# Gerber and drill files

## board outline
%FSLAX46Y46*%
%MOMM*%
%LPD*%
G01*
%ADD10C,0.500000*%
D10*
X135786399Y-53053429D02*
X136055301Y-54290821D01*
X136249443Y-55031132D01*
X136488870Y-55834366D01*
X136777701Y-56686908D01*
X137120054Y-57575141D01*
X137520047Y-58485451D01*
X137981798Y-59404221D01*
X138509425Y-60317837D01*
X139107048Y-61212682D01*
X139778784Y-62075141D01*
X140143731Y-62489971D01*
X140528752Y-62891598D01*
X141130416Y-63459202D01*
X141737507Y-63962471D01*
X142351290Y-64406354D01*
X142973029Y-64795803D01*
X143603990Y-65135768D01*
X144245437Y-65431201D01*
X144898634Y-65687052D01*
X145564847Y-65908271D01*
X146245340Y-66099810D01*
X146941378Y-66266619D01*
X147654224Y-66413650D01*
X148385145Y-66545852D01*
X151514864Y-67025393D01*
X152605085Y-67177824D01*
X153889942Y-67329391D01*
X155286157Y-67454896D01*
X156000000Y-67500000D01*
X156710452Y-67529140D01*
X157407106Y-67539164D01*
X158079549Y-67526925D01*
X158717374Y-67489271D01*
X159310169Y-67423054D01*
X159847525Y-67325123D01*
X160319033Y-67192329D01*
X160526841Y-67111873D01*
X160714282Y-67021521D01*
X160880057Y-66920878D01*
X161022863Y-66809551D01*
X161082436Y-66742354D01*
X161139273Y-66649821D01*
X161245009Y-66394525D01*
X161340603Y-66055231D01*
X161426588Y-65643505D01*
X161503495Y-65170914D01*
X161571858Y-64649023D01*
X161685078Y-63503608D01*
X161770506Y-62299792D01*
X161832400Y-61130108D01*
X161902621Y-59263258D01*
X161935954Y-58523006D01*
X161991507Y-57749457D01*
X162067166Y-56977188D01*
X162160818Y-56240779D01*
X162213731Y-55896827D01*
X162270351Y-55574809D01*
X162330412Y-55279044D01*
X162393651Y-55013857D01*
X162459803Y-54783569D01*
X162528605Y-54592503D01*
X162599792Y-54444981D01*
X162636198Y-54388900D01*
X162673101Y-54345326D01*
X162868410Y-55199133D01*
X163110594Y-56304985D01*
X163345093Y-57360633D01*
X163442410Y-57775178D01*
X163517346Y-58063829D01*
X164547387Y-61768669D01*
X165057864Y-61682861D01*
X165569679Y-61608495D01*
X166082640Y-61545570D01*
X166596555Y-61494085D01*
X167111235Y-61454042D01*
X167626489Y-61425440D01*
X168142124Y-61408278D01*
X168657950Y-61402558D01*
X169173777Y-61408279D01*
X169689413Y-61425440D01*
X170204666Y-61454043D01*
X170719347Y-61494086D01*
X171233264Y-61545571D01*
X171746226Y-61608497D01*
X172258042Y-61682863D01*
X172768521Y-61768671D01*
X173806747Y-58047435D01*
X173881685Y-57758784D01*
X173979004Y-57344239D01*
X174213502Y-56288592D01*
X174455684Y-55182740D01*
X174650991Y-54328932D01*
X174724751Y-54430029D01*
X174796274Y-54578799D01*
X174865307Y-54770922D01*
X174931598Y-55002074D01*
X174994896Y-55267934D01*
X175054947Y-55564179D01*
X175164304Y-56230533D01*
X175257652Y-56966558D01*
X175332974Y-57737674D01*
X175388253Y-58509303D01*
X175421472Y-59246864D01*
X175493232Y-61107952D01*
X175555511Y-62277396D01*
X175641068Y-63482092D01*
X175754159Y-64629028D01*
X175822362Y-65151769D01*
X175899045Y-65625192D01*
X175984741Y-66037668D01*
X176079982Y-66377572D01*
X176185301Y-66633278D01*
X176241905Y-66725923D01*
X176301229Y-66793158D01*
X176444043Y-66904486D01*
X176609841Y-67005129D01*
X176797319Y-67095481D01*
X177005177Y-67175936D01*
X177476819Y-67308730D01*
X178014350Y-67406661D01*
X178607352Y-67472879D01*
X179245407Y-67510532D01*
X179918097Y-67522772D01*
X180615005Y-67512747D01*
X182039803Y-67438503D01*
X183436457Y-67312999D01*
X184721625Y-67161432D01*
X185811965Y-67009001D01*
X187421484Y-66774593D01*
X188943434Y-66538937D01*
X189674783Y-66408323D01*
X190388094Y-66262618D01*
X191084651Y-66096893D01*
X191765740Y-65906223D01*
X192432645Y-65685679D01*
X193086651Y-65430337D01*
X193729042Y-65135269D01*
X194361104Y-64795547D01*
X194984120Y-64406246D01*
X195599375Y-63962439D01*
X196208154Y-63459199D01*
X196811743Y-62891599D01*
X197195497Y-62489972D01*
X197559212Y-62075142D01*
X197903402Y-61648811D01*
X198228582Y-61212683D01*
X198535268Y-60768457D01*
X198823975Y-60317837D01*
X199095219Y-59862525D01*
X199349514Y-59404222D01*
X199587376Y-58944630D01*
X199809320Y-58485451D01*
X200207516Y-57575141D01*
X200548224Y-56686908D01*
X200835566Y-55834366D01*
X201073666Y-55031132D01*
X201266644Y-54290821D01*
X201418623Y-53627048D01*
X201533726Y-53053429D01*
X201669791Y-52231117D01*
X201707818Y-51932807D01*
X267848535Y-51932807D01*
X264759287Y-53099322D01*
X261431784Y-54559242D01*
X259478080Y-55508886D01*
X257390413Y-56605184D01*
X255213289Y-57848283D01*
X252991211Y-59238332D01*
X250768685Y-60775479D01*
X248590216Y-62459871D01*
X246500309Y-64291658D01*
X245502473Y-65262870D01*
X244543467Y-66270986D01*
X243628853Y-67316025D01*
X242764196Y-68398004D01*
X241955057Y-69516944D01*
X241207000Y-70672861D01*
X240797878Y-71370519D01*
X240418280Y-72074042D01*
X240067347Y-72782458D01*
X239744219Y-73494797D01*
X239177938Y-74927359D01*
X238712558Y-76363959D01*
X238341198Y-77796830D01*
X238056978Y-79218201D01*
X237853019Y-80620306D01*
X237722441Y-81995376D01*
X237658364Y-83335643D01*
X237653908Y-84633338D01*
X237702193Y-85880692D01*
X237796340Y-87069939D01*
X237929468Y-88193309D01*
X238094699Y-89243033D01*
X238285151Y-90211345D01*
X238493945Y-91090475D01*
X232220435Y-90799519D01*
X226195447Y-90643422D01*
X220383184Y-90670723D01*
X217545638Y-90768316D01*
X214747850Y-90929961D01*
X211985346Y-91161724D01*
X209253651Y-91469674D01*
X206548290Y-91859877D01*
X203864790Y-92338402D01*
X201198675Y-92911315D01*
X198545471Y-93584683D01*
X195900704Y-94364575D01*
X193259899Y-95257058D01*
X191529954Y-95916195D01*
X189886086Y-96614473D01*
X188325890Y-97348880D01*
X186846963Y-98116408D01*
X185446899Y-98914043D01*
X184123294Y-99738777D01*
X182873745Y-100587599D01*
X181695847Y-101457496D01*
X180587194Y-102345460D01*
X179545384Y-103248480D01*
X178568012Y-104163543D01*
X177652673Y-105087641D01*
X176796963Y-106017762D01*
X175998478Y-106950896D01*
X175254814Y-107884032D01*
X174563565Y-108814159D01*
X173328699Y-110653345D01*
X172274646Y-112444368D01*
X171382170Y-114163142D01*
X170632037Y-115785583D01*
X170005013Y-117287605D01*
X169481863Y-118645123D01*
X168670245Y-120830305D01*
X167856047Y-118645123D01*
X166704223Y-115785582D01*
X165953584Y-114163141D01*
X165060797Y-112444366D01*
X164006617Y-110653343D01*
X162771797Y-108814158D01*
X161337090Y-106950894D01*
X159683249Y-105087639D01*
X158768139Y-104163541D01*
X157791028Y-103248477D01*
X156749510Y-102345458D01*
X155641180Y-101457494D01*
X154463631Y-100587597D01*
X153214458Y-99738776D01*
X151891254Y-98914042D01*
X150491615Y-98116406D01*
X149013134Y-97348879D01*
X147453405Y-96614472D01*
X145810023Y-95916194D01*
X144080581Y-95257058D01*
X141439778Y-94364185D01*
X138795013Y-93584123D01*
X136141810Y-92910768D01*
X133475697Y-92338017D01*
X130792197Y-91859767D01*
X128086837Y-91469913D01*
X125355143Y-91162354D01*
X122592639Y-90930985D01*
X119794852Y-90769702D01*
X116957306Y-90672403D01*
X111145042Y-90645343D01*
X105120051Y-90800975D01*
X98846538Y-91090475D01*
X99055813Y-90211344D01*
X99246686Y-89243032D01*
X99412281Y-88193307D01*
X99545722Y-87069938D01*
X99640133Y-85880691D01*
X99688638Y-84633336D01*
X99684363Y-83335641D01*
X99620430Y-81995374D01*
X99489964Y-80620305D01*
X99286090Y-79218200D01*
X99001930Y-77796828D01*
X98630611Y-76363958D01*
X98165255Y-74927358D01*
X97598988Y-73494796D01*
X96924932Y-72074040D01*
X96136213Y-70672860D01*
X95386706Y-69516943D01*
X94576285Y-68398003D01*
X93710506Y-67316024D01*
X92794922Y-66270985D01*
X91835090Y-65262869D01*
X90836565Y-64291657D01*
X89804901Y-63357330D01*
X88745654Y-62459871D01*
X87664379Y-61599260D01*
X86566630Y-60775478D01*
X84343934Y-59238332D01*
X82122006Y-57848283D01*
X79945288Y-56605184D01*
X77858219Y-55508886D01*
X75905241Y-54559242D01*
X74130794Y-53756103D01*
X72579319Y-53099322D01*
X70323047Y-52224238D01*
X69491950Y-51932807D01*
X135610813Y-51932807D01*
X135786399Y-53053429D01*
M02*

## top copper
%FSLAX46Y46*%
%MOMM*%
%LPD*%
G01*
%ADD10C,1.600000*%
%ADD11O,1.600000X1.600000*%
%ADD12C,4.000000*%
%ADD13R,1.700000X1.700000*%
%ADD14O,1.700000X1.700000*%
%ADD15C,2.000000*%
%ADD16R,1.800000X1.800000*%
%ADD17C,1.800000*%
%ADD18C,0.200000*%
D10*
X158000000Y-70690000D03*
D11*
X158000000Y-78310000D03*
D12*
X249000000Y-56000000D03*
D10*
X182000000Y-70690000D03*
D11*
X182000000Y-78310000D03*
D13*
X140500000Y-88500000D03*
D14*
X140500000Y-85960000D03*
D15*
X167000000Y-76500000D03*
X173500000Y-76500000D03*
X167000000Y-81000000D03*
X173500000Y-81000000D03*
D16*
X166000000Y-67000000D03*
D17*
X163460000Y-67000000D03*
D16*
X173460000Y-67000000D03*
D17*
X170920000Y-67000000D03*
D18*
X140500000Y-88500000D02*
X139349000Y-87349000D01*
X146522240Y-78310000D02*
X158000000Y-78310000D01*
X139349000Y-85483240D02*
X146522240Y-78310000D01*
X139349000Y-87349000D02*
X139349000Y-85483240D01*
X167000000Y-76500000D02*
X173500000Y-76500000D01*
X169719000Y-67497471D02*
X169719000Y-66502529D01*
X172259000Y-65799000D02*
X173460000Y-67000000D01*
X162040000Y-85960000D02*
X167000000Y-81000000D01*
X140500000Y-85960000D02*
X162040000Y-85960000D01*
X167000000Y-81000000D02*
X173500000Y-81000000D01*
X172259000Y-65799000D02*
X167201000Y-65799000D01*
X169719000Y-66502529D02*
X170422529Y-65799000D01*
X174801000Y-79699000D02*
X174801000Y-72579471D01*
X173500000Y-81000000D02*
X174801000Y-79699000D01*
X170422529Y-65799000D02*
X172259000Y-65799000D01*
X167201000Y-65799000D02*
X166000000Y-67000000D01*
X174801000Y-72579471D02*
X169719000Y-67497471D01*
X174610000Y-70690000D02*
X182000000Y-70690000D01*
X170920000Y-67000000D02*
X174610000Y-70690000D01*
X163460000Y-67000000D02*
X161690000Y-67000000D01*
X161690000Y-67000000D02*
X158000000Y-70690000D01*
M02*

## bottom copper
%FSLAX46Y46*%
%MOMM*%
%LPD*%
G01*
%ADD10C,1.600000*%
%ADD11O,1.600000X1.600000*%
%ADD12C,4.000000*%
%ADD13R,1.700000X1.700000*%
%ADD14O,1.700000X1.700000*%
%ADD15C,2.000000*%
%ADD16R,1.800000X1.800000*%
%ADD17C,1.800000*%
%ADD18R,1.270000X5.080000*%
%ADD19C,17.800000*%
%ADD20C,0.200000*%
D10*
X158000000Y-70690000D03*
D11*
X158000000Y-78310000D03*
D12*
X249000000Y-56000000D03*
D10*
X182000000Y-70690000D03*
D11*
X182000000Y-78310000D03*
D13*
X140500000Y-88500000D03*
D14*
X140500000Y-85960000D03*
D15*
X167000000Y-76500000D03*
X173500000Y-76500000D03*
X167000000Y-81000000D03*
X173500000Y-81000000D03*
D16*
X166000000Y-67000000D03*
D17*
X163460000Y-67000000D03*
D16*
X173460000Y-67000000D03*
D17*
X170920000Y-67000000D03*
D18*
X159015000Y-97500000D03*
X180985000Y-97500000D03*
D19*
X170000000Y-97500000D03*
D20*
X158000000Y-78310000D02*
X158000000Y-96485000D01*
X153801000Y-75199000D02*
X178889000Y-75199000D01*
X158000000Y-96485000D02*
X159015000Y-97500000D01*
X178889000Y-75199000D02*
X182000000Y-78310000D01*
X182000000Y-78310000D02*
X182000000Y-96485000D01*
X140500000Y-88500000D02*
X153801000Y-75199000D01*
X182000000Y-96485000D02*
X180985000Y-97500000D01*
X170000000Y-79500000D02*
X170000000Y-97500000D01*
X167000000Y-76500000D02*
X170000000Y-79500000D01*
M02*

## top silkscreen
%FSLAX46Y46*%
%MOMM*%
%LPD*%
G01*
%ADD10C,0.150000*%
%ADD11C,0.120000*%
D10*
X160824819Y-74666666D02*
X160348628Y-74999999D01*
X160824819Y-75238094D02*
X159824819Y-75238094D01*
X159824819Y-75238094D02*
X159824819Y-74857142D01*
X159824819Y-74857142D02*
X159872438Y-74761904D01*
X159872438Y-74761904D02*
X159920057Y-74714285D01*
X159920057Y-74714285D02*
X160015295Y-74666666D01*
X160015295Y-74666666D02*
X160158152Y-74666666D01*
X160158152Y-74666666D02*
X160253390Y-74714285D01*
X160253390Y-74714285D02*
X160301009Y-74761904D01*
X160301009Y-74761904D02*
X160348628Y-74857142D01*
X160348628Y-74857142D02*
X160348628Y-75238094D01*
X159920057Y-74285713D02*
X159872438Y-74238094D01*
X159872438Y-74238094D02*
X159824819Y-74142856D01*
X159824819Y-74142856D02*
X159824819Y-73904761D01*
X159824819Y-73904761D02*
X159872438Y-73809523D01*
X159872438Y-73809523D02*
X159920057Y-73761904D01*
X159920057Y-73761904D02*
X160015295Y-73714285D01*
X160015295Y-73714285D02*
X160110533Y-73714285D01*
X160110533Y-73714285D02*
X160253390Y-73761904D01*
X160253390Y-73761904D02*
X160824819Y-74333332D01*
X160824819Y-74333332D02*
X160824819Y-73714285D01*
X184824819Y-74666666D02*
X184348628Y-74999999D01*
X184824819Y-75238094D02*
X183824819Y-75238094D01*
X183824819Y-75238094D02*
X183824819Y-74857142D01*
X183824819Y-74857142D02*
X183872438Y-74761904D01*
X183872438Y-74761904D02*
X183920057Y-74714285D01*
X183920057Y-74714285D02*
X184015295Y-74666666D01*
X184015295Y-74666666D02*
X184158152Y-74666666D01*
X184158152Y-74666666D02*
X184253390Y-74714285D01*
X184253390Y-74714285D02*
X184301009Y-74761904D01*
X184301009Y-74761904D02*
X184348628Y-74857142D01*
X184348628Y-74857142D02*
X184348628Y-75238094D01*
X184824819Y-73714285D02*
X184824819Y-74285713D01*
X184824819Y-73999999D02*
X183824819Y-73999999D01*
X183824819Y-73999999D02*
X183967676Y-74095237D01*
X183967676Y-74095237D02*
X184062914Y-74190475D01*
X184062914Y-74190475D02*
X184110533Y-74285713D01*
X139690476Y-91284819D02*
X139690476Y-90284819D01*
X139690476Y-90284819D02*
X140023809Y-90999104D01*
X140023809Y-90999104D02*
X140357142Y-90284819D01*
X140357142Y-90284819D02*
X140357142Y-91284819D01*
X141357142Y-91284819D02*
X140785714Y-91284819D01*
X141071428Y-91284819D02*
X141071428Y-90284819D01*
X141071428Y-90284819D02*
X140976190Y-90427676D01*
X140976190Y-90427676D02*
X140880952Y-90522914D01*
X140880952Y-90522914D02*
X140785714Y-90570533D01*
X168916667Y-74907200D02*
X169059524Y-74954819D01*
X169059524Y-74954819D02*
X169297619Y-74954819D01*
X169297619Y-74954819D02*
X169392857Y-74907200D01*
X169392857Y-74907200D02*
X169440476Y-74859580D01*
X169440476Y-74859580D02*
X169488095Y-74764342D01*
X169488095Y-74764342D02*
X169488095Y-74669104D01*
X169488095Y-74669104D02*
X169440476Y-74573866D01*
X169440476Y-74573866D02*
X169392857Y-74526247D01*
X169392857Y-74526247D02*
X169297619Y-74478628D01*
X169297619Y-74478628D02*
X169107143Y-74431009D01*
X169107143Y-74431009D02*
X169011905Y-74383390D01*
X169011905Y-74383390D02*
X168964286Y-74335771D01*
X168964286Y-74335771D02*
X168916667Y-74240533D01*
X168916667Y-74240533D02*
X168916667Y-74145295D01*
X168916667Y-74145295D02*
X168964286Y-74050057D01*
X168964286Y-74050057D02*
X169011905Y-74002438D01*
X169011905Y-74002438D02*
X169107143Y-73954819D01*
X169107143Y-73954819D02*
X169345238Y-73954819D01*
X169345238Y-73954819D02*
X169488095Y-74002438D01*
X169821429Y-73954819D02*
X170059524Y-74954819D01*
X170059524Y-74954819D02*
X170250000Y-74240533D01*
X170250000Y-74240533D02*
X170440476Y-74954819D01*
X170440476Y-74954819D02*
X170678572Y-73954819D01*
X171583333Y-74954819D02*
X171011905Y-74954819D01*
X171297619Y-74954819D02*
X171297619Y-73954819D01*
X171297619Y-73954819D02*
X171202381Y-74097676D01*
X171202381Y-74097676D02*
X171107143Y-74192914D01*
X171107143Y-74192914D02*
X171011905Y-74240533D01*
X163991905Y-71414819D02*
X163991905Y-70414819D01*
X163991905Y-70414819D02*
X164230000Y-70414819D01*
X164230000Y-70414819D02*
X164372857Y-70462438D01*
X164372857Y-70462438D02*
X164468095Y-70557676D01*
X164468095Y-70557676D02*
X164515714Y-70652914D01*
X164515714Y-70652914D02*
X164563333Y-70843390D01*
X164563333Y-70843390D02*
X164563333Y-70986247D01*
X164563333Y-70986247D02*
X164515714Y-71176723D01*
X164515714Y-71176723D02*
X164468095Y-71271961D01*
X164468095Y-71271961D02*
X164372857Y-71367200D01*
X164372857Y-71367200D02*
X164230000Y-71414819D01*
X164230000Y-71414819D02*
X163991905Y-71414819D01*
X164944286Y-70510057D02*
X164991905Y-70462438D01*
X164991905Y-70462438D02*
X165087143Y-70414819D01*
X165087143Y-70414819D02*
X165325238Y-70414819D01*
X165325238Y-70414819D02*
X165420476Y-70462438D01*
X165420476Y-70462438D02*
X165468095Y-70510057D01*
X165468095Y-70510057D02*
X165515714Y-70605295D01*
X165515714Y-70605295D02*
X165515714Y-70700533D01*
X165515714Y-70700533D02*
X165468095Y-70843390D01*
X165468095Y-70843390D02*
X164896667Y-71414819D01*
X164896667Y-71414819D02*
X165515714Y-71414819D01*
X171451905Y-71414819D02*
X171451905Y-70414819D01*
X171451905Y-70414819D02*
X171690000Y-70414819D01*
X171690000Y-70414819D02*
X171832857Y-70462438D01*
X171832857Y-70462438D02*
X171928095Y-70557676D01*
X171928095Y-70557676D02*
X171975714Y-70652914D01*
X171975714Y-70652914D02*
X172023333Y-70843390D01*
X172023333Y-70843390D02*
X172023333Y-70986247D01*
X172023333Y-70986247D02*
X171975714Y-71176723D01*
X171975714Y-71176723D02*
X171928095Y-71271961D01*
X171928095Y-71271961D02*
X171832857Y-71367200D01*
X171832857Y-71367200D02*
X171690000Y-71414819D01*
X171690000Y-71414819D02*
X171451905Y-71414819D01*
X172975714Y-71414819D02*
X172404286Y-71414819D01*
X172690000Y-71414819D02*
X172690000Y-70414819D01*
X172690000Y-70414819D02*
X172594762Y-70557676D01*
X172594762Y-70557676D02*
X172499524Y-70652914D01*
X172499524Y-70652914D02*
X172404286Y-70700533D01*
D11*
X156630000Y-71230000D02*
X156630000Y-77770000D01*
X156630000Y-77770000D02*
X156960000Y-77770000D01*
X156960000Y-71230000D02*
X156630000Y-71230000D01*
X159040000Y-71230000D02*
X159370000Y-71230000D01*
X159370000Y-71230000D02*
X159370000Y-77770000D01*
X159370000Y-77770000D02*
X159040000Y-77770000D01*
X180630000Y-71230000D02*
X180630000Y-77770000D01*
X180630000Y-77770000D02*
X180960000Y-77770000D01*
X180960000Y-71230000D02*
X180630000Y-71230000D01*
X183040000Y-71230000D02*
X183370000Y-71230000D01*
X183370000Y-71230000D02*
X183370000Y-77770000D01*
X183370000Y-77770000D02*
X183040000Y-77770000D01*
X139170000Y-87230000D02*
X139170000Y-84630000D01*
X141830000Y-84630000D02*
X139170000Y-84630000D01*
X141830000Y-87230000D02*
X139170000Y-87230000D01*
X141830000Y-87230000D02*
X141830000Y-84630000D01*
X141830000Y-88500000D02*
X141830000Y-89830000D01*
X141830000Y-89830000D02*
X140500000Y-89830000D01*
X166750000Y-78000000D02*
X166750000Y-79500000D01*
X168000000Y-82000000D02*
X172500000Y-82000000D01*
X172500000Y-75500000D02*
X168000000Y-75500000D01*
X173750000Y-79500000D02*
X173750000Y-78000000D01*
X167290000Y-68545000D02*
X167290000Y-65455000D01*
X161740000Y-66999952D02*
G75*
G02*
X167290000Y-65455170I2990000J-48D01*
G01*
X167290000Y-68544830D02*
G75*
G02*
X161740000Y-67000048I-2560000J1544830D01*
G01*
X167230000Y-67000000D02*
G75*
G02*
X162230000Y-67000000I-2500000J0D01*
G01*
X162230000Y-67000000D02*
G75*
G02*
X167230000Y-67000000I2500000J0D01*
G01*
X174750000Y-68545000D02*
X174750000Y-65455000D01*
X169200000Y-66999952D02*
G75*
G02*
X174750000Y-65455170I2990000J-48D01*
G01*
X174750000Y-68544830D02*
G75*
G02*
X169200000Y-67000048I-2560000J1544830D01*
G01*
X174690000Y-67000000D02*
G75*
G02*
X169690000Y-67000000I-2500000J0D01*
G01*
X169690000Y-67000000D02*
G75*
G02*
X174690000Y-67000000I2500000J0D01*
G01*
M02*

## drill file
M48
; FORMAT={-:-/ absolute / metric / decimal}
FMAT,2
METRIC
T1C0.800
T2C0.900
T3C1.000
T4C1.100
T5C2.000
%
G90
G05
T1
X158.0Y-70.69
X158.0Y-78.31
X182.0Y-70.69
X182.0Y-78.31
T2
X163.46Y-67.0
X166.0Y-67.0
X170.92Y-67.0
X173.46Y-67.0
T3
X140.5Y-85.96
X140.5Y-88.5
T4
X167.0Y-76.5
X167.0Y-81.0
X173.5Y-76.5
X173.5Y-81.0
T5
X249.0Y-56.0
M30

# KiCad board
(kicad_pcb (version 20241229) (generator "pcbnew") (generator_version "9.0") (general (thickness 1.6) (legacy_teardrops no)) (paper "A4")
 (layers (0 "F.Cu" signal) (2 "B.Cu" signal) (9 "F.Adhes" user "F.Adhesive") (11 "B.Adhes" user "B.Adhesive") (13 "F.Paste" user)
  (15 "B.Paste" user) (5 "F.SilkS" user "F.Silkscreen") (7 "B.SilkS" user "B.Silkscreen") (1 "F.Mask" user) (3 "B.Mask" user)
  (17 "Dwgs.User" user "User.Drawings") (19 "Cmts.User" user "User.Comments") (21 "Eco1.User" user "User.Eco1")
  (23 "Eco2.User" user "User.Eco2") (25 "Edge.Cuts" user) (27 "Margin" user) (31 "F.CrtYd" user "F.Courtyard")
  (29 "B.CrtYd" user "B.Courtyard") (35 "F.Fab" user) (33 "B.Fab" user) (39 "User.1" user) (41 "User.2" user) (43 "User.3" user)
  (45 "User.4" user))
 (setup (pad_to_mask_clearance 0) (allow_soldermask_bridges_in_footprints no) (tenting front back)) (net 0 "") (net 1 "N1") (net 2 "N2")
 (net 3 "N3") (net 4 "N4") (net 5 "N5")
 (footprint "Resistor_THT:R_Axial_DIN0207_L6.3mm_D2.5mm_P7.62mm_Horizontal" (layer "F.Cu") (at 158 70.69 -90)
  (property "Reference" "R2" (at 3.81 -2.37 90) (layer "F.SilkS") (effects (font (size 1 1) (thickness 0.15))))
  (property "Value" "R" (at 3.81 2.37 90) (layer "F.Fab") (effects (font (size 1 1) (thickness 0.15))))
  (fp_line (start 0.54 1.37) (end 7.08 1.37) (stroke (width 0.12) (type solid)) (layer "F.SilkS"))
  (fp_line (start 7.08 1.37) (end 7.08 1.04) (stroke (width 0.12) (type solid)) (layer "F.SilkS"))
  (fp_line (start 0.54 1.04) (end 0.54 1.37) (stroke (width 0.12) (type solid)) (layer "F.SilkS"))
  (fp_line (start 0.54 -1.04) (end 0.54 -1.37) (stroke (width 0.12) (type solid)) (layer "F.SilkS"))
  (fp_line (start 0.54 -1.37) (end 7.08 -1.37) (stroke (width 0.12) (type solid)) (layer "F.SilkS"))
  (fp_line (start 7.08 -1.37) (end 7.08 -1.04) (stroke (width 0.12) (type solid)) (layer "F.SilkS"))
  (pad "1" thru_hole circle (at 0 0 270) (size 1.6 1.6) (drill 0.8) (layers "*.Cu" "*.Mask") (remove_unused_layers no) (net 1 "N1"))
  (pad "2" thru_hole oval (at 7.62 0 270) (size 1.6 1.6) (drill 0.8) (layers "*.Cu" "*.Mask") (remove_unused_layers no) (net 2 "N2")))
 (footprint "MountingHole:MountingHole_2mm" (layer "F.Cu") (at 249 56)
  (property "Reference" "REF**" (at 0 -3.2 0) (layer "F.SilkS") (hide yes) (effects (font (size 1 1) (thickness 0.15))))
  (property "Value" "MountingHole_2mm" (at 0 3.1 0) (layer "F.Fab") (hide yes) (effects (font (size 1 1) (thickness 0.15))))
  (pad "" np_thru_hole circle (at 0 0) (size 4 4) (drill 2) (layers "*.Cu" "*.Mask")))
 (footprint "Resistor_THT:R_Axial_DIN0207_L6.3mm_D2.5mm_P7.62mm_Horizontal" (layer "F.Cu") (at 182 70.69 -90)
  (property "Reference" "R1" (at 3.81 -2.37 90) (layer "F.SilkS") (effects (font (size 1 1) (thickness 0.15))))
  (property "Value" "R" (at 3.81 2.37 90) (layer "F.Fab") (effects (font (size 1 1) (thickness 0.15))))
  (fp_line (start 0.54 1.37) (end 7.08 1.37) (stroke (width 0.12) (type solid)) (layer "F.SilkS"))
  (fp_line (start 7.08 1.37) (end 7.08 1.04) (stroke (width 0.12) (type solid)) (layer "F.SilkS"))
  (fp_line (start 0.54 1.04) (end 0.54 1.37) (stroke (width 0.12) (type solid)) (layer "F.SilkS"))
  (fp_line (start 0.54 -1.04) (end 0.54 -1.37) (stroke (width 0.12) (type solid)) (layer "F.SilkS"))
  (fp_line (start 0.54 -1.37) (end 7.08 -1.37) (stroke (width 0.12) (type solid)) (layer "F.SilkS"))
  (fp_line (start 7.08 -1.37) (end 7.08 -1.04) (stroke (width 0.12) (type solid)) (layer "F.SilkS"))
  (pad "1" thru_hole circle (at 0 0 270) (size 1.6 1.6) (drill 0.8) (layers "*.Cu" "*.Mask") (remove_unused_layers no) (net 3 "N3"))
  (pad "2" thru_hole oval (at 7.62 0 270) (size 1.6 1.6) (drill 0.8) (layers "*.Cu" "*.Mask") (remove_unused_layers no) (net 2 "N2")))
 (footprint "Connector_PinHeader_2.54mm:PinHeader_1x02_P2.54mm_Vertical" (layer "F.Cu") (at 140.5 88.5 180)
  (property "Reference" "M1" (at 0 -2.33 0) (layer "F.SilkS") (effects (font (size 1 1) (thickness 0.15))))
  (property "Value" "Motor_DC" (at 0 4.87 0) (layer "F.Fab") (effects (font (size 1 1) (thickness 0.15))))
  (fp_line (start 1.33 1.27) (end 1.33 3.87) (stroke (width 0.12) (type solid)) (layer "F.SilkS"))
  (fp_line (start -1.33 3.87) (end 1.33 3.87) (stroke (width 0.12) (type solid)) (layer "F.SilkS"))
  (fp_line (start -1.33 1.27) (end 1.33 1.27) (stroke (width 0.12) (type solid)) (layer "F.SilkS"))
  (fp_line (start -1.33 1.27) (end -1.33 3.87) (stroke (width 0.12) (type solid)) (layer "F.SilkS"))
  (fp_line (start -1.33 0) (end -1.33 -1.33) (stroke (width 0.12) (type solid)) (layer "F.SilkS"))
  (fp_line (start -1.33 -1.33) (end 0 -1.33) (stroke (width 0.12) (type solid)) (layer "F.SilkS"))
  (pad "1" thru_hole rect (at 0 0 180) (size 1.7 1.7) (drill 1) (layers "*.Cu" "*.Mask") (remove_unused_layers no) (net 2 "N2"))
  (pad "2" thru_hole oval (at 0 2.54 180) (size 1.7 1.7) (drill 1) (layers "*.Cu" "*.Mask") (remove_unused_layers no) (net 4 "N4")))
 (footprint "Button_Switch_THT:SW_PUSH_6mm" (layer "F.Cu") (at 167 76.5)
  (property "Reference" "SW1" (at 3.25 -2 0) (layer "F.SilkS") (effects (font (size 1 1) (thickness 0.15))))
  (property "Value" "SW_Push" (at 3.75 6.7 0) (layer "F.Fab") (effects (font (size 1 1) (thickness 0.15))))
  (fp_line (start -0.25 1.5) (end -0.25 3) (stroke (width 0.12) (type solid)) (layer "F.SilkS"))
  (fp_line (start 1 5.5) (end 5.5 5.5) (stroke (width 0.12) (type solid)) (layer "F.SilkS"))
  (fp_line (start 5.5 -1) (end 1 -1) (stroke (width 0.12) (type solid)) (layer "F.SilkS"))
  (fp_line (start 6.75 3) (end 6.75 1.5) (stroke (width 0.12) (type solid)) (layer "F.SilkS"))
  (pad "1" thru_hole circle (at 0 0 90) (size 2 2) (drill 1.1) (layers "*.Cu" "*.Mask") (remove_unused_layers no) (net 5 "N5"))
  (pad "1" thru_hole circle (at 6.5 0 90) (size 2 2) (drill 1.1) (layers "*.Cu" "*.Mask") (remove_unused_layers no) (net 5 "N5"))
  (pad "2" thru_hole circle (at 0 4.5 90) (size 2 2) (drill 1.1) (layers "*.Cu" "*.Mask") (remove_unused_layers no) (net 4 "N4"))
  (pad "2" thru_hole circle (at 6.5 4.5 90) (size 2 2) (drill 1.1) (layers "*.Cu" "*.Mask") (remove_unused_layers no) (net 4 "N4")))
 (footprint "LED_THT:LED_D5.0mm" (layer "F.Cu") (at 166 67 180)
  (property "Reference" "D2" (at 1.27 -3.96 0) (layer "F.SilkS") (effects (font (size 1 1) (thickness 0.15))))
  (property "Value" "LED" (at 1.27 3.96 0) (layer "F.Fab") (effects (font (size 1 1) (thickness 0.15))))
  (fp_line (start -1.29 -1.545) (end -1.29 1.545) (stroke (width 0.12) (type solid)) (layer "F.SilkS"))
  (fp_arc (start 4.26 0.000048) (mid 2.071756 2.880501) (end -1.29 1.54483) (stroke (width 0.12) (type solid)) (layer "F.SilkS"))
  (fp_arc (start -1.29 -1.54483) (mid 2.071756 -2.880501) (end 4.26 -0.000048) (stroke (width 0.12) (type solid)) (layer "F.SilkS"))
  (fp_circle (center 1.27 0) (end 3.77 0) (stroke (width 0.12) (type solid)) (fill no) (layer "F.SilkS"))
  (pad "1" thru_hole rect (at 0 0 180) (size 1.8 1.8) (drill 0.9) (layers "*.Cu" "*.Mask") (remove_unused_layers no) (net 4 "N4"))
  (pad "2" thru_hole circle (at 2.54 0 180) (size 1.8 1.8) (drill 0.9) (layers "*.Cu" "*.Mask") (remove_unused_layers no) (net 1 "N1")))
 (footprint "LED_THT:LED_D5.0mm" (layer "F.Cu") (at 173.46 67 180)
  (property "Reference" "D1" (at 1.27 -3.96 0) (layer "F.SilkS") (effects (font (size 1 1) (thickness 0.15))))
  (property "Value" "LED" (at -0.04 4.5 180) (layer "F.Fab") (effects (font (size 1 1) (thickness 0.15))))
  (fp_line (start -1.29 -1.545) (end -1.29 1.545) (stroke (width 0.12) (type solid)) (layer "F.SilkS"))
  (fp_arc (start 4.26 0.000048) (mid 2.071756 2.880501) (end -1.29 1.54483) (stroke (width 0.12) (type solid)) (layer "F.SilkS"))
  (fp_arc (start -1.29 -1.54483) (mid 2.071756 -2.880501) (end 4.26 -0.000048) (stroke (width 0.12) (type solid)) (layer "F.SilkS"))
  (fp_circle (center 1.27 0) (end 3.77 0) (stroke (width 0.12) (type solid)) (fill no) (layer "F.SilkS"))
  (pad "1" thru_hole rect (at 0 0 180) (size 1.8 1.8) (drill 0.9) (layers "*.Cu" "*.Mask") (remove_unused_layers no) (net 4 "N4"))
  (pad "2" thru_hole circle (at 2.54 0 180) (size 1.8 1.8) (drill 0.9) (layers "*.Cu" "*.Mask") (remove_unused_layers no) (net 3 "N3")))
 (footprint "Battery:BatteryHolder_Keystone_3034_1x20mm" (layer "B.Cu") (at 170 97.5)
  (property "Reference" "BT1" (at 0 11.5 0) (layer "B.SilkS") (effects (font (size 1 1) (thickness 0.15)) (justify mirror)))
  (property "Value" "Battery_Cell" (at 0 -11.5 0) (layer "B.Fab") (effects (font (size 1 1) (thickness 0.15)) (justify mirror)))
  (pad "1" smd rect (at -10.985 0) (size 1.27 5.08) (layers "B.Cu" "B.Mask" "B.Paste") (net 2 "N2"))
  (pad "1" smd rect (at 10.985 0) (size 1.27 5.08) (layers "B.Cu" "B.Mask" "B.Paste") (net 2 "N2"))
  (pad "2" smd circle (at 0 0) (size 17.8 17.8) (layers "B.Cu" "B.Mask") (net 5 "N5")))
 (gr_poly
  (pts (xy 135.786399 53.053429) (xy 136.055301 54.290821) (xy 136.249443 55.031132) (xy 136.48887 55.834366) (xy 136.777701 56.686908)
   (xy 137.120054 57.575141) (xy 137.520047 58.485451) (xy 137.981798 59.404221) (xy 138.509425 60.317837) (xy 139.107048 61.212682)
   (xy 139.778784 62.075141) (xy 140.143731 62.489971) (xy 140.528752 62.891598) (xy 141.130416 63.459202) (xy 141.737507 63.962471)
   (xy 142.35129 64.406354) (xy 142.973029 64.795803) (xy 143.60399 65.135768) (xy 144.245437 65.431201) (xy 144.898634 65.687052)
   (xy 145.564847 65.908271) (xy 146.24534 66.09981) (xy 146.941378 66.266619) (xy 147.654224 66.41365) (xy 148.385145 66.545852)
   (xy 151.514864 67.025393) (xy 152.605085 67.177824) (xy 153.889942 67.329391) (xy 155.286157 67.454896) (xy 156 67.5)
   (xy 156.710452 67.52914) (xy 157.407106 67.539164) (xy 158.079549 67.526925) (xy 158.717374 67.489271) (xy 159.310169 67.423054)
   (xy 159.847525 67.325123) (xy 160.319033 67.192329) (xy 160.526841 67.111873) (xy 160.714282 67.021521) (xy 160.880057 66.920878)
   (xy 161.022863 66.809551) (xy 161.082436 66.742354) (xy 161.139273 66.649821) (xy 161.245009 66.394525) (xy 161.340603 66.055231)
   (xy 161.426588 65.643505) (xy 161.503495 65.170914) (xy 161.571858 64.649023) (xy 161.685078 63.503608) (xy 161.770506 62.299792)
   (xy 161.8324 61.130108) (xy 161.902621 59.263258) (xy 161.935954 58.523006) (xy 161.991507 57.749457) (xy 162.067166 56.977188)
   (xy 162.160818 56.240779) (xy 162.213731 55.896827) (xy 162.270351 55.574809) (xy 162.330412 55.279044) (xy 162.393651 55.013857)
   (xy 162.459803 54.783569) (xy 162.528605 54.592503) (xy 162.599792 54.444981) (xy 162.636198 54.3889) (xy 162.673101 54.345326)
   (xy 162.86841 55.199133) (xy 163.110594 56.304985) (xy 163.345093 57.360633) (xy 163.44241 57.775178) (xy 163.517346 58.063829)
   (xy 164.547387 61.768669) (xy 165.057864 61.682861) (xy 165.569679 61.608495) (xy 166.08264 61.54557) (xy 166.596555 61.494085)
   (xy 167.111235 61.454042) (xy 167.626489 61.42544) (xy 168.142124 61.408278) (xy 168.65795 61.402558) (xy 169.173777 61.408279)
   (xy 169.689413 61.42544) (xy 170.204666 61.454043) (xy 170.719347 61.494086) (xy 171.233264 61.545571) (xy 171.746226 61.608497)
   (xy 172.258042 61.682863) (xy 172.768521 61.768671) (xy 173.806747 58.047435) (xy 173.881685 57.758784) (xy 173.979004 57.344239)
   (xy 174.213502 56.288592) (xy 174.455684 55.18274) (xy 174.650991 54.328932) (xy 174.724751 54.430029) (xy 174.796274 54.578799)
   (xy 174.865307 54.770922) (xy 174.931598 55.002074) (xy 174.994896 55.267934) (xy 175.054947 55.564179) (xy 175.164304 56.230533)
   (xy 175.257652 56.966558) (xy 175.332974 57.737674) (xy 175.388253 58.509303) (xy 175.421472 59.246864) (xy 175.493232 61.107952)
   (xy 175.555511 62.277396) (xy 175.641068 63.482092) (xy 175.754159 64.629028) (xy 175.822362 65.151769) (xy 175.899045 65.625192)
   (xy 175.984741 66.037668) (xy 176.079982 66.377572) (xy 176.185301 66.633278) (xy 176.241905 66.725923) (xy 176.301229 66.793158)
   (xy 176.444043 66.904486) (xy 176.609841 67.005129) (xy 176.797319 67.095481) (xy 177.005177 67.175936) (xy 177.476819 67.30873)
   (xy 178.01435 67.406661) (xy 178.607352 67.472879) (xy 179.245407 67.510532) (xy 179.918097 67.522772) (xy 180.615005 67.512747)
   (xy 182.039803 67.438503) (xy 183.436457 67.312999) (xy 184.721625 67.161432) (xy 185.811965 67.009001) (xy 187.421484 66.774593)
   (xy 188.943434 66.538937) (xy 189.674783 66.408323) (xy 190.388094 66.262618) (xy 191.084651 66.096893) (xy 191.76574 65.906223)
   (xy 192.432645 65.685679) (xy 193.086651 65.430337) (xy 193.729042 65.135269) (xy 194.361104 64.795547) (xy 194.98412 64.406246)
   (xy 195.599375 63.962439) (xy 196.208154 63.459199) (xy 196.811743 62.891599) (xy 197.195497 62.489972) (xy 197.559212 62.075142)
   (xy 197.903402 61.648811) (xy 198.228582 61.212683) (xy 198.535268 60.768457) (xy 198.823975 60.317837) (xy 199.095219 59.862525)
   (xy 199.349514 59.404222) (xy 199.587376 58.94463) (xy 199.80932 58.485451) (xy 200.207516 57.575141) (xy 200.548224 56.686908)
   (xy 200.835566 55.834366) (xy 201.073666 55.031132) (xy 201.266644 54.290821) (xy 201.418623 53.627048) (xy 201.533726 53.053429)
   (xy 201.669791 52.231117) (xy 201.707818 51.932807) (xy 267.848535 51.932807) (xy 264.759287 53.099322) (xy 261.431784 54.559242)
   (xy 259.47808 55.508886) (xy 257.390413 56.605184) (xy 255.213289 57.848283) (xy 252.991211 59.238332) (xy 250.768685 60.775479)
   (xy 248.590216 62.459871) (xy 246.500309 64.291658) (xy 245.502473 65.26287) (xy 244.543467 66.270986) (xy 243.628853 67.316025)
   (xy 242.764196 68.398004) (xy 241.955057 69.516944) (xy 241.207 70.672861) (xy 240.797878 71.370519) (xy 240.41828 72.074042)
   (xy 240.067347 72.782458) (xy 239.744219 73.494797) (xy 239.177938 74.927359) (xy 238.712558 76.363959) (xy 238.341198 77.79683)
   (xy 238.056978 79.218201) (xy 237.853019 80.620306) (xy 237.722441 81.995376) (xy 237.658364 83.335643) (xy 237.653908 84.633338)
   (xy 237.702193 85.880692) (xy 237.79634 87.069939) (xy 237.929468 88.193309) (xy 238.094699 89.243033) (xy 238.285151 90.211345)
   (xy 238.493945 91.090475) (xy 232.220435 90.799519) (xy 226.195447 90.643422) (xy 220.383184 90.670723) (xy 217.545638 90.768316)
   (xy 214.74785 90.929961) (xy 211.985346 91.161724) (xy 209.253651 91.469674) (xy 206.54829 91.859877) (xy 203.86479 92.338402)
   (xy 201.198675 92.911315) (xy 198.545471 93.584683) (xy 195.900704 94.364575) (xy 193.259899 95.257058) (xy 191.529954 95.916195)
   (xy 189.886086 96.614473) (xy 188.32589 97.34888) (xy 186.846963 98.116408) (xy 185.446899 98.914043) (xy 184.123294 99.738777)
   (xy 182.873745 100.587599) (xy 181.695847 101.457496) (xy 180.587194 102.34546) (xy 179.545384 103.24848) (xy 178.568012 104.163543)
   (xy 177.652673 105.087641) (xy 176.796963 106.017762) (xy 175.998478 106.950896) (xy 175.254814 107.884032) (xy 174.563565 108.814159)
   (xy 173.328699 110.653345) (xy 172.274646 112.444368) (xy 171.38217 114.163142) (xy 170.632037 115.785583) (xy 170.005013 117.287605)
   (xy 169.481863 118.645123) (xy 168.670245 120.830305) (xy 167.856047 118.645123) (xy 166.704223 115.785582) (xy 165.953584 114.163141)
   (xy 165.060797 112.444366) (xy 164.006617 110.653343) (xy 162.771797 108.814158) (xy 161.33709 106.950894) (xy 159.683249 105.087639)
   (xy 158.768139 104.163541) (xy 157.791028 103.248477) (xy 156.74951 102.345458) (xy 155.64118 101.457494) (xy 154.463631 100.587597)
   (xy 153.214458 99.738776) (xy 151.891254 98.914042) (xy 150.491615 98.116406) (xy 149.013134 97.348879) (xy 147.453405 96.614472)
   (xy 145.810023 95.916194) (xy 144.080581 95.257058) (xy 141.439778 94.364185) (xy 138.795013 93.584123) (xy 136.14181 92.910768)
   (xy 133.475697 92.338017) (xy 130.792197 91.859767) (xy 128.086837 91.469913) (xy 125.355143 91.162354) (xy 122.592639 90.930985)
   (xy 119.794852 90.769702) (xy 116.957306 90.672403) (xy 111.145042 90.645343) (xy 105.120051 90.800975) (xy 98.846538 91.090475)
   (xy 99.055813 90.211344) (xy 99.246686 89.243032) (xy 99.412281 88.193307) (xy 99.545722 87.069938) (xy 99.640133 85.880691)
   (xy 99.688638 84.633336) (xy 99.684363 83.335641) (xy 99.62043 81.995374) (xy 99.489964 80.620305) (xy 99.28609 79.2182)
   (xy 99.00193 77.796828) (xy 98.630611 76.363958) (xy 98.165255 74.927358) (xy 97.598988 73.494796) (xy 96.924932 72.07404)
   (xy 96.136213 70.67286) (xy 95.386706 69.516943) (xy 94.576285 68.398003) (xy 93.710506 67.316024) (xy 92.794922 66.270985)
   (xy 91.83509 65.262869) (xy 90.836565 64.291657) (xy 89.804901 63.35733) (xy 88.745654 62.459871) (xy 87.664379 61.59926)
   (xy 86.56663 60.775478) (xy 84.343934 59.238332) (xy 82.122006 57.848283) (xy 79.945288 56.605184) (xy 77.858219 55.508886)
   (xy 75.905241 54.559242) (xy 74.130794 53.756103) (xy 72.579319 53.099322) (xy 70.323047 52.224238) (xy 69.49195 51.932807)
   (xy 135.610813 51.932807))
  (stroke (width 0.5) (type solid)) (fill no) (layer "Edge.Cuts"))
 (segment (start 140.5 88.5) (end 139.349 87.349) (width 0.2) (layer "F.Cu") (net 2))
 (segment (start 146.52224 78.31) (end 158 78.31) (width 0.2) (layer "F.Cu") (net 2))
 (segment (start 139.349 85.48324) (end 146.52224 78.31) (width 0.2) (layer "F.Cu") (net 2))
 (segment (start 139.349 87.349) (end 139.349 85.48324) (width 0.2) (layer "F.Cu") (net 2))
 (segment (start 158 78.31) (end 158 96.485) (width 0.2) (layer "B.Cu") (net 2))
 (segment (start 153.801 75.199) (end 178.889 75.199) (width 0.2) (layer "B.Cu") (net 2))
 (segment (start 158 96.485) (end 159.015 97.5) (width 0.2) (layer "B.Cu") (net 2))
 (segment (start 178.889 75.199) (end 182 78.31) (width 0.2) (layer "B.Cu") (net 2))
 (segment (start 182 78.31) (end 182 96.485) (width 0.2) (layer "B.Cu") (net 2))
 (segment (start 140.5 88.5) (end 153.801 75.199) (width 0.2) (layer "B.Cu") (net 2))
 (segment (start 182 96.485) (end 180.985 97.5) (width 0.2) (layer "B.Cu") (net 2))
 (segment (start 167 76.5) (end 173.5 76.5) (width 0.2) (layer "F.Cu") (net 5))
 (segment (start 170 79.5) (end 170 97.5) (width 0.2) (layer "B.Cu") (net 5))
 (segment (start 167 76.5) (end 170 79.5) (width 0.2) (layer "B.Cu") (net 5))
 (segment (start 169.719 67.497471) (end 169.719 66.502529) (width 0.2) (layer "F.Cu") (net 4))
 (segment (start 172.259 65.799) (end 173.46 67) (width 0.2) (layer "F.Cu") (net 4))
 (segment (start 162.04 85.96) (end 167 81) (width 0.2) (layer "F.Cu") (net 4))
 (segment (start 140.5 85.96) (end 162.04 85.96) (width 0.2) (layer "F.Cu") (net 4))
 (segment (start 167 81) (end 173.5 81) (width 0.2) (layer "F.Cu") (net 4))
 (segment (start 172.259 65.799) (end 167.201 65.799) (width 0.2) (layer "F.Cu") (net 4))
 (segment (start 169.719 66.502529) (end 170.422529 65.799) (width 0.2) (layer "F.Cu") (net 4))
 (segment (start 174.801 79.699) (end 174.801 72.579471) (width 0.2) (layer "F.Cu") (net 4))
 (segment (start 173.5 81) (end 174.801 79.699) (width 0.2) (layer "F.Cu") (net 4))
 (segment (start 170.422529 65.799) (end 172.259 65.799) (width 0.2) (layer "F.Cu") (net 4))
 (segment (start 167.201 65.799) (end 166 67) (width 0.2) (layer "F.Cu") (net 4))
 (segment (start 174.801 72.579471) (end 169.719 67.497471) (width 0.2) (layer "F.Cu") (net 4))
 (segment (start 174.61 70.69) (end 182 70.69) (width 0.2) (layer "F.Cu") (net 3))
 (segment (start 170.92 67) (end 174.61 70.69) (width 0.2) (layer "F.Cu") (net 3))
 (segment (start 163.46 67) (end 161.69 67) (width 0.2) (layer "F.Cu") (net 1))
 (segment (start 161.69 67) (end 158 70.69) (width 0.2) (layer "F.Cu") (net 1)))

